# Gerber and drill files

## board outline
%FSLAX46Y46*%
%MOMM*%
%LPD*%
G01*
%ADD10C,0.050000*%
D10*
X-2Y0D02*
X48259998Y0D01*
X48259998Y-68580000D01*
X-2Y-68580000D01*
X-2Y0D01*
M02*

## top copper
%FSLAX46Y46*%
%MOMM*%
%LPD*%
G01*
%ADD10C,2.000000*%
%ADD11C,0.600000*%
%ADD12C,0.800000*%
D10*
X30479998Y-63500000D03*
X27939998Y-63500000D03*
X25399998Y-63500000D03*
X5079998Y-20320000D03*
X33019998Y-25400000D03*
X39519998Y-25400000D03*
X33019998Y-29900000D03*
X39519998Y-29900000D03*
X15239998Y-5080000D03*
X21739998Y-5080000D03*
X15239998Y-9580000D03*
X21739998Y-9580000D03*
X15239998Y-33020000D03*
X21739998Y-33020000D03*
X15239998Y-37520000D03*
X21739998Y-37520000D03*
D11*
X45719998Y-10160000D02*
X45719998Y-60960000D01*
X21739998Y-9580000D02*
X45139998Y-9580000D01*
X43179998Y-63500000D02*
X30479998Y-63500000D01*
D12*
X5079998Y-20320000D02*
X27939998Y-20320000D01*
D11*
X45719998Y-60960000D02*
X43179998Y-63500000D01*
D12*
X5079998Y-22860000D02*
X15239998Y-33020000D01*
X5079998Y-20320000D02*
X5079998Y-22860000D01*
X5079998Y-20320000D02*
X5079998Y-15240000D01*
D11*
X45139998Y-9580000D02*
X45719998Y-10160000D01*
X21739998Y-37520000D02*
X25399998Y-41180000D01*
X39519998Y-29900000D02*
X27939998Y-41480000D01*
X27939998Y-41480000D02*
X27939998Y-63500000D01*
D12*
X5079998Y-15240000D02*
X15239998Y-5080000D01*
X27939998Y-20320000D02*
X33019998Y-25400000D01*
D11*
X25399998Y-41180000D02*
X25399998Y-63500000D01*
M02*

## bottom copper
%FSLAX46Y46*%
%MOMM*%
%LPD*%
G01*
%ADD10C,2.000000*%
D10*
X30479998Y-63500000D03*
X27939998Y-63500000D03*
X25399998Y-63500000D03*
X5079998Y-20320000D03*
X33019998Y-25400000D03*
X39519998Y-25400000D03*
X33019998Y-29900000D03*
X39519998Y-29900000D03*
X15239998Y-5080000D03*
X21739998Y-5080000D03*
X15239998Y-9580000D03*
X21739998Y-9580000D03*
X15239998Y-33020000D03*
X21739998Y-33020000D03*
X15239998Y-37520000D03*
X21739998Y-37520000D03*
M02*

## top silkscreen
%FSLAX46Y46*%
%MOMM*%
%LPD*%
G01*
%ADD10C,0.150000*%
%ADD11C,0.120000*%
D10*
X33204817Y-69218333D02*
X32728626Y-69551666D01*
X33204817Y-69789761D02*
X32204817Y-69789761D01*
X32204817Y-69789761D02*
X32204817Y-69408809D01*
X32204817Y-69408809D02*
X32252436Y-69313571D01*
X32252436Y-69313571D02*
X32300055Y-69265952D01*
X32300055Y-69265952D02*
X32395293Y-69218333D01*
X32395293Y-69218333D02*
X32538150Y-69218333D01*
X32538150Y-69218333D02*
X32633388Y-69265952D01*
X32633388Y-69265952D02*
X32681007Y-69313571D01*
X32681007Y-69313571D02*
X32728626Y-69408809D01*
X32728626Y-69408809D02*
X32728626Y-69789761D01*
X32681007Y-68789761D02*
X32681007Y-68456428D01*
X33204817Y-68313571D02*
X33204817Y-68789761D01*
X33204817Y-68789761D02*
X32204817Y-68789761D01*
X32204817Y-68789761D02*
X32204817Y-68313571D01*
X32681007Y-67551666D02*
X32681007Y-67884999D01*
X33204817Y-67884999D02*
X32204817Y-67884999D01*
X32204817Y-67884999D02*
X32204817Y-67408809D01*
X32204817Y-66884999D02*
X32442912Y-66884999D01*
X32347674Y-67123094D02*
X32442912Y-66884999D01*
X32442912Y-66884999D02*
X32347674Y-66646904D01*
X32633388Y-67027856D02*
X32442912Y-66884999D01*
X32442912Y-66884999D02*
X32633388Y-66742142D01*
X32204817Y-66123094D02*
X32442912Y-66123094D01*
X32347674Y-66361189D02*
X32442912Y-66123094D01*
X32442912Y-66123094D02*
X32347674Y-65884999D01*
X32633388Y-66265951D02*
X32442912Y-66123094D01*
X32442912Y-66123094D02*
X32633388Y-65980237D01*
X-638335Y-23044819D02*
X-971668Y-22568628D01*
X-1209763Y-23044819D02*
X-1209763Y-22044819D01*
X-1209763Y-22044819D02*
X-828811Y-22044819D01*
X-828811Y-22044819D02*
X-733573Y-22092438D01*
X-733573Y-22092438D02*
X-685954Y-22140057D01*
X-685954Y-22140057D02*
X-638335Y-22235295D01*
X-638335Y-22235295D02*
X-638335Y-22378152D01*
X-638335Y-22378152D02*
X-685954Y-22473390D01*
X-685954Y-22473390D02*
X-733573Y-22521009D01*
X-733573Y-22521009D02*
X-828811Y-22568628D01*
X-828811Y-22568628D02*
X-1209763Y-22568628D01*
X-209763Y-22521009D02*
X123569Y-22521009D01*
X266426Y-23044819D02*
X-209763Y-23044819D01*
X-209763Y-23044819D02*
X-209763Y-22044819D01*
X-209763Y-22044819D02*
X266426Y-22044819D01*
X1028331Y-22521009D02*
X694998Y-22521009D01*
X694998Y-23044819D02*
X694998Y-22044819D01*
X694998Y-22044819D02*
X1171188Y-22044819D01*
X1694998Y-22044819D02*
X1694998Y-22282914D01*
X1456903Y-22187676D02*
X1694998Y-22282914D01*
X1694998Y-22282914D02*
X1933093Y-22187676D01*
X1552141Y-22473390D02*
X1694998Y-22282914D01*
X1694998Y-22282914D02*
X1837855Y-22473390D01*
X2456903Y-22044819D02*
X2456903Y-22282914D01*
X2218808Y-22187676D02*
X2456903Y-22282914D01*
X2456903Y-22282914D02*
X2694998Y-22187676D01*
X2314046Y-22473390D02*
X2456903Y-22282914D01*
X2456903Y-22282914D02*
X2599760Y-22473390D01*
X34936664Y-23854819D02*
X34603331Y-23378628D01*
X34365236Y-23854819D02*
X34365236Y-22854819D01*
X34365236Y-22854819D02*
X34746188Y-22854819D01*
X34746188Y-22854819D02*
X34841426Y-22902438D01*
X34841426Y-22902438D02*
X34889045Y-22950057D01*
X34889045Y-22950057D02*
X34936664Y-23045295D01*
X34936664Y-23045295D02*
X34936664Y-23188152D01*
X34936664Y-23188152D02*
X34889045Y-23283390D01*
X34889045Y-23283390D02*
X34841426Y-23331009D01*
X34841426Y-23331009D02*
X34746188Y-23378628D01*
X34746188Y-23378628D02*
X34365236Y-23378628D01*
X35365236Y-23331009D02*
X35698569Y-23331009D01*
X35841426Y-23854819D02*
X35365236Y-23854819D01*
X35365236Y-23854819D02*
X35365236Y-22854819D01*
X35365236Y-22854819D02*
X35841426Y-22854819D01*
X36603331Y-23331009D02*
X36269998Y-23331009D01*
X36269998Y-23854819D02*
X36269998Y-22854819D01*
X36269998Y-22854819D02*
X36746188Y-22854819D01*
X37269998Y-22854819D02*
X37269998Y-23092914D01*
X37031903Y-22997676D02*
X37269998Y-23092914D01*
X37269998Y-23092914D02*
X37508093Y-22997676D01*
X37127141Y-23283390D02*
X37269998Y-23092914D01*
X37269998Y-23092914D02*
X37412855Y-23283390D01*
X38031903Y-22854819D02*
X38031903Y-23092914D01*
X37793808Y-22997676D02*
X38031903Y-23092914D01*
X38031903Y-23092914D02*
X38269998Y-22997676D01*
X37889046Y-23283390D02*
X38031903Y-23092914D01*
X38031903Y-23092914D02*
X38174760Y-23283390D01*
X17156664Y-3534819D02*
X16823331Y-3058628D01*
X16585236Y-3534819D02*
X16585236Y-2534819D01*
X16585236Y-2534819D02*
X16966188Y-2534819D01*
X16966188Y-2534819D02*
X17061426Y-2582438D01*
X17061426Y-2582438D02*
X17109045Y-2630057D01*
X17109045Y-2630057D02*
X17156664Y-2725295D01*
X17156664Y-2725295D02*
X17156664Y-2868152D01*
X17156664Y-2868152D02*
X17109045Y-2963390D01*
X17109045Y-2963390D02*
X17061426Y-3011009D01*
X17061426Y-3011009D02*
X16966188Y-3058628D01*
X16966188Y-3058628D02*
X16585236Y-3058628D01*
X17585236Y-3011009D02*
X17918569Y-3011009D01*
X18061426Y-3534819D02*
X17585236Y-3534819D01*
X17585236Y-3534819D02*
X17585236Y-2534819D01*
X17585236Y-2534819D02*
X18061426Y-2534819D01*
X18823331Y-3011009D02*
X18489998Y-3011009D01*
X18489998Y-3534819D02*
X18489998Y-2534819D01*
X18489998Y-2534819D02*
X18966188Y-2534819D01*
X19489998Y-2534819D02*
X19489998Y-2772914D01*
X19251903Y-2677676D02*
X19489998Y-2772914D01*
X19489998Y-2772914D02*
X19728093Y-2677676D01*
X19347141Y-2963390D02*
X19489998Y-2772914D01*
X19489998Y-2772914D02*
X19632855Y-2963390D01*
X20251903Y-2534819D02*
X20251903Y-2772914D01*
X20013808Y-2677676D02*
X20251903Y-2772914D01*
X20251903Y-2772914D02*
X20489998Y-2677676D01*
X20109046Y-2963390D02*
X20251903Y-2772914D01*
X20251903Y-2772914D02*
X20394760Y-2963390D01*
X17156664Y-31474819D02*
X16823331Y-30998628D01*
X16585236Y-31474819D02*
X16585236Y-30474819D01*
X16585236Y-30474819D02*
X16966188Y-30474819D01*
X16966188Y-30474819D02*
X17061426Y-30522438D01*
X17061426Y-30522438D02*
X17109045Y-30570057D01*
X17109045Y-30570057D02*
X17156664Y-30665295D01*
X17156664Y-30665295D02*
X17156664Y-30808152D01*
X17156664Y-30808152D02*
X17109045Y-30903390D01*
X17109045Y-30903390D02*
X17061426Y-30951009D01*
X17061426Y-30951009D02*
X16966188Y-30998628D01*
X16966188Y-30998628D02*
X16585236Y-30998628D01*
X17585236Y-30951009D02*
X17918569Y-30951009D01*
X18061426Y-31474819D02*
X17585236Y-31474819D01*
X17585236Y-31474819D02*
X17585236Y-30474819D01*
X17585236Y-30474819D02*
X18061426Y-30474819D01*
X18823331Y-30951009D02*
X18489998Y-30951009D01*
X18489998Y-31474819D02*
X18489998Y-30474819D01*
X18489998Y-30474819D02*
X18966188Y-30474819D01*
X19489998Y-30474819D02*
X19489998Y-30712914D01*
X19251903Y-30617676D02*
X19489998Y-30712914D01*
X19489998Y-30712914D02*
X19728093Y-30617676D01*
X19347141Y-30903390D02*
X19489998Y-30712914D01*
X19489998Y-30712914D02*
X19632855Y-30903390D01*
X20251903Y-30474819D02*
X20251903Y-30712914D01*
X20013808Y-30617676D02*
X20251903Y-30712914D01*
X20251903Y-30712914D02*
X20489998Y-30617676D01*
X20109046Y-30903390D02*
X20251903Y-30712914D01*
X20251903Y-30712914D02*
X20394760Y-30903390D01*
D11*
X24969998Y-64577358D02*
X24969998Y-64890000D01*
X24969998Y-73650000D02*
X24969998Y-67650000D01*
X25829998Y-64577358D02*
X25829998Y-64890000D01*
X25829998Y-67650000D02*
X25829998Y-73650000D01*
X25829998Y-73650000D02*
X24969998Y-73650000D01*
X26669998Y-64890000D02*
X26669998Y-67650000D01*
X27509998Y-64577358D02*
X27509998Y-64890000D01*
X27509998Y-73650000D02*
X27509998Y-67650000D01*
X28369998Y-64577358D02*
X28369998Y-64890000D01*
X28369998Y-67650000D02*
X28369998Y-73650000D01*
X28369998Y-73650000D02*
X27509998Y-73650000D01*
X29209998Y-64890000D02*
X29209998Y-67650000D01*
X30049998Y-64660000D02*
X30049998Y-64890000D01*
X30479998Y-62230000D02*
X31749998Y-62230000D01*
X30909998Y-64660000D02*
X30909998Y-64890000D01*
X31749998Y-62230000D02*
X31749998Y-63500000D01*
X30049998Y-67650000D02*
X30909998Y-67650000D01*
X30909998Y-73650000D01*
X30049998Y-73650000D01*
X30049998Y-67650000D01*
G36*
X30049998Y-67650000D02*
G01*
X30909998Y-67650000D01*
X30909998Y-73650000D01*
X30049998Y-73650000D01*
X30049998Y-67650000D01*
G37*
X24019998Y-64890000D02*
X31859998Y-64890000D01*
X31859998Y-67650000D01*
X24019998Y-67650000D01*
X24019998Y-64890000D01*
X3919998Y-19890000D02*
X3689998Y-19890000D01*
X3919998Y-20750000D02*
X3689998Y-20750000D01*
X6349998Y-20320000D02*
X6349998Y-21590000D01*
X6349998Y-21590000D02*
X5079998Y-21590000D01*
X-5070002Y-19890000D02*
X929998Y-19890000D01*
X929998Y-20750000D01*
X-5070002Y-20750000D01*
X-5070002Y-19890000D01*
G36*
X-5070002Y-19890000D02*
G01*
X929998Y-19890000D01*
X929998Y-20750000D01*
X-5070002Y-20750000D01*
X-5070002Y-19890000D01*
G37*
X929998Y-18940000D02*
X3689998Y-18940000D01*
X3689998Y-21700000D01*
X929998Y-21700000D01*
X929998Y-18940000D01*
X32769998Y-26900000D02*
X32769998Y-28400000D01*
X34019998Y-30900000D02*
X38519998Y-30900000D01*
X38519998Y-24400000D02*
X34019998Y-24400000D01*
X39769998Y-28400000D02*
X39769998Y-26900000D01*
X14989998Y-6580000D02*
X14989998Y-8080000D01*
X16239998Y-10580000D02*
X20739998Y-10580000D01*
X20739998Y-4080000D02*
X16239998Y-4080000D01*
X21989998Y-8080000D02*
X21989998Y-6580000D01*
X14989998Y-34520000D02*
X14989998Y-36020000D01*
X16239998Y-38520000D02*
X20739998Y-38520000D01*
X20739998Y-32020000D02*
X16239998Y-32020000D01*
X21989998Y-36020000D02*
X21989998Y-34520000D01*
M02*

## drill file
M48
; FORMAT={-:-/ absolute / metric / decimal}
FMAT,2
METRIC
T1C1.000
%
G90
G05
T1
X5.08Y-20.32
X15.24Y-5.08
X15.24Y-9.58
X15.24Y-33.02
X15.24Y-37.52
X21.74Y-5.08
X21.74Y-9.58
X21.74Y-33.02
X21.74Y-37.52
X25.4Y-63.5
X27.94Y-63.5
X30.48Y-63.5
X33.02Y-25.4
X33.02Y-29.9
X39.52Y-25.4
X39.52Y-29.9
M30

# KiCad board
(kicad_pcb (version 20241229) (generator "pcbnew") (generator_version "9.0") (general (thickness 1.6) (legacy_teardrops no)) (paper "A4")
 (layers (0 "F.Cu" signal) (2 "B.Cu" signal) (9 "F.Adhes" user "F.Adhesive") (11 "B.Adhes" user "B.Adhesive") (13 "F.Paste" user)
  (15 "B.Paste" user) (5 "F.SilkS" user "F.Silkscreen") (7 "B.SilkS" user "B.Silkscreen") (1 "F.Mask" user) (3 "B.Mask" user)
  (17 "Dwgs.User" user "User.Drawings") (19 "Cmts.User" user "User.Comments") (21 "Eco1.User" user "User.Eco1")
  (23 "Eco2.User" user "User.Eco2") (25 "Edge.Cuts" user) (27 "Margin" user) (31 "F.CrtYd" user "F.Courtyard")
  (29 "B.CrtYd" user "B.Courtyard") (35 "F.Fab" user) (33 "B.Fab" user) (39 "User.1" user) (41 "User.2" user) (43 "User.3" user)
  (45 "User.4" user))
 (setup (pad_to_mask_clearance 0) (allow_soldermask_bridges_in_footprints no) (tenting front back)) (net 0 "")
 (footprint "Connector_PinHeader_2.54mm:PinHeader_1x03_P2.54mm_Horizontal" (layer "F.Cu") (at 30.479998 63.5 -90)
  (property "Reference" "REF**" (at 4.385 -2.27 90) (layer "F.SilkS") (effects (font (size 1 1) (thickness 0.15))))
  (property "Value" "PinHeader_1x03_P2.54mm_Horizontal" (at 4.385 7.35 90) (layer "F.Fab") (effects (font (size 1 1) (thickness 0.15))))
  (fp_line (start 1.077358 5.51) (end 1.39 5.51) (stroke (width 0.12) (type solid)) (layer "F.SilkS"))
  (fp_line (start 10.15 5.51) (end 4.15 5.51) (stroke (width 0.12) (type solid)) (layer "F.SilkS"))
  (fp_line (start 1.077358 4.65) (end 1.39 4.65) (stroke (width 0.12) (type solid)) (layer "F.SilkS"))
  (fp_line (start 4.15 4.65) (end 10.15 4.65) (stroke (width 0.12) (type solid)) (layer "F.SilkS"))
  (fp_line (start 10.15 4.65) (end 10.15 5.51) (stroke (width 0.12) (type solid)) (layer "F.SilkS"))
  (fp_line (start 1.39 3.81) (end 4.15 3.81) (stroke (width 0.12) (type solid)) (layer "F.SilkS"))
  (fp_line (start 1.077358 2.97) (end 1.39 2.97) (stroke (width 0.12) (type solid)) (layer "F.SilkS"))
  (fp_line (start 10.15 2.97) (end 4.15 2.97) (stroke (width 0.12) (type solid)) (layer "F.SilkS"))
  (fp_line (start 1.077358 2.11) (end 1.39 2.11) (stroke (width 0.12) (type solid)) (layer "F.SilkS"))
  (fp_line (start 4.15 2.11) (end 10.15 2.11) (stroke (width 0.12) (type solid)) (layer "F.SilkS"))
  (fp_line (start 10.15 2.11) (end 10.15 2.97) (stroke (width 0.12) (type solid)) (layer "F.SilkS"))
  (fp_line (start 1.39 1.27) (end 4.15 1.27) (stroke (width 0.12) (type solid)) (layer "F.SilkS"))
  (fp_line (start 1.16 0.43) (end 1.39 0.43) (stroke (width 0.12) (type solid)) (layer "F.SilkS"))
  (fp_line (start -1.27 0) (end -1.27 -1.27) (stroke (width 0.12) (type solid)) (layer "F.SilkS"))
  (fp_line (start 1.16 -0.43) (end 1.39 -0.43) (stroke (width 0.12) (type solid)) (layer "F.SilkS"))
  (fp_line (start -1.27 -1.27) (end 0 -1.27) (stroke (width 0.12) (type solid)) (layer "F.SilkS"))
  (fp_rect (start 4.15 -0.43) (end 10.15 0.43) (stroke (width 0.12) (type solid)) (fill yes) (layer "F.SilkS"))
  (fp_rect (start 1.39 -1.38) (end 4.15 6.46) (stroke (width 0.12) (type solid)) (fill no) (layer "F.SilkS"))
  (pad "1" thru_hole circle (at 0 0 270) (size 2 2) (drill 1) (layers "*.Cu" "*.Mask") (remove_unused_layers no))
  (pad "2" thru_hole circle (at 0 2.54 270) (size 2 2) (drill 1) (layers "*.Cu" "*.Mask") (remove_unused_layers no))
  (pad "3" thru_hole circle (at 0 5.08 270) (size 2 2) (drill 1) (layers "*.Cu" "*.Mask") (remove_unused_layers no)))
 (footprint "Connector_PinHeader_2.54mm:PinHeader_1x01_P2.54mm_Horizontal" (layer "F.Cu") (at 5.079998 20.32 180)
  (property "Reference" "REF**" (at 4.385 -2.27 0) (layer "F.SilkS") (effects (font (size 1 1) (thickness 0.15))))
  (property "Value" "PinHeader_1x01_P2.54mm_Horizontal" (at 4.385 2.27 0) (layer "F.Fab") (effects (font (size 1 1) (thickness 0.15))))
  (fp_line (start 1.16 0.43) (end 1.39 0.43) (stroke (width 0.12) (type solid)) (layer "F.SilkS"))
  (fp_line (start 1.16 -0.43) (end 1.39 -0.43) (stroke (width 0.12) (type solid)) (layer "F.SilkS"))
  (fp_line (start -1.27 0) (end -1.27 -1.27) (stroke (width 0.12) (type solid)) (layer "F.SilkS"))
  (fp_line (start -1.27 -1.27) (end 0 -1.27) (stroke (width 0.12) (type solid)) (layer "F.SilkS"))
  (fp_rect (start 4.15 -0.43) (end 10.15 0.43) (stroke (width 0.12) (type solid)) (fill yes) (layer "F.SilkS"))
  (fp_rect (start 1.39 -1.38) (end 4.15 1.38) (stroke (width 0.12) (type solid)) (fill no) (layer "F.SilkS"))
  (pad "1" thru_hole circle (at 0 0 180) (size 2 2) (drill 1) (layers "*.Cu" "*.Mask") (remove_unused_layers no)))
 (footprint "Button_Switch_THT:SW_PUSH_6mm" (layer "F.Cu") (at 33.019998 25.4)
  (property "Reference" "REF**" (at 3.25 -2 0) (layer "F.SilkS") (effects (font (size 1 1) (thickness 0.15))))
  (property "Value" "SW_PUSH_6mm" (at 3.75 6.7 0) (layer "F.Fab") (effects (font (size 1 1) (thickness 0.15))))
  (fp_line (start -0.25 1.5) (end -0.25 3) (stroke (width 0.12) (type solid)) (layer "F.SilkS"))
  (fp_line (start 1 5.5) (end 5.5 5.5) (stroke (width 0.12) (type solid)) (layer "F.SilkS"))
  (fp_line (start 5.5 -1) (end 1 -1) (stroke (width 0.12) (type solid)) (layer "F.SilkS"))
  (fp_line (start 6.75 3) (end 6.75 1.5) (stroke (width 0.12) (type solid)) (layer "F.SilkS"))
  (pad "1" thru_hole circle (at 0 0 90) (size 2 2) (drill 1) (layers "*.Cu" "*.Mask") (remove_unused_layers no))
  (pad "1" thru_hole circle (at 6.5 0 90) (size 2 2) (drill 1) (layers "*.Cu" "*.Mask") (remove_unused_layers no))
  (pad "2" thru_hole circle (at 0 4.5 90) (size 2 2) (drill 1) (layers "*.Cu" "*.Mask") (remove_unused_layers no))
  (pad "2" thru_hole circle (at 6.5 4.5 90) (size 2 2) (drill 1) (layers "*.Cu" "*.Mask") (remove_unused_layers no)))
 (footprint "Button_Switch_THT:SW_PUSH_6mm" (layer "F.Cu") (at 15.239998 5.08)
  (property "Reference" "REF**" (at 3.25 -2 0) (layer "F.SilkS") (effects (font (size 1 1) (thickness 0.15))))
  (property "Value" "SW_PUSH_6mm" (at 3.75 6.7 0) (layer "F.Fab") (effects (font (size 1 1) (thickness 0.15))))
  (fp_line (start -0.25 1.5) (end -0.25 3) (stroke (width 0.12) (type solid)) (layer "F.SilkS"))
  (fp_line (start 1 5.5) (end 5.5 5.5) (stroke (width 0.12) (type solid)) (layer "F.SilkS"))
  (fp_line (start 5.5 -1) (end 1 -1) (stroke (width 0.12) (type solid)) (layer "F.SilkS"))
  (fp_line (start 6.75 3) (end 6.75 1.5) (stroke (width 0.12) (type solid)) (layer "F.SilkS"))
  (pad "1" thru_hole circle (at 0 0 90) (size 2 2) (drill 1) (layers "*.Cu" "*.Mask") (remove_unused_layers no))
  (pad "1" thru_hole circle (at 6.5 0 90) (size 2 2) (drill 1) (layers "*.Cu" "*.Mask") (remove_unused_layers no))
  (pad "2" thru_hole circle (at 0 4.5 90) (size 2 2) (drill 1) (layers "*.Cu" "*.Mask") (remove_unused_layers no))
  (pad "2" thru_hole circle (at 6.5 4.5 90) (size 2 2) (drill 1) (layers "*.Cu" "*.Mask") (remove_unused_layers no)))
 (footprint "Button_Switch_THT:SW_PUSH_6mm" (layer "F.Cu") (at 15.239998 33.02)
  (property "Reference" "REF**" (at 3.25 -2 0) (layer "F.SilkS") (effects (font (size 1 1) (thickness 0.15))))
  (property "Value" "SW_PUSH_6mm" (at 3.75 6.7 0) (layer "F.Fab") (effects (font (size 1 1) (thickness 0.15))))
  (fp_line (start -0.25 1.5) (end -0.25 3) (stroke (width 0.12) (type solid)) (layer "F.SilkS"))
  (fp_line (start 1 5.5) (end 5.5 5.5) (stroke (width 0.12) (type solid)) (layer "F.SilkS"))
  (fp_line (start 5.5 -1) (end 1 -1) (stroke (width 0.12) (type solid)) (layer "F.SilkS"))
  (fp_line (start 6.75 3) (end 6.75 1.5) (stroke (width 0.12) (type solid)) (layer "F.SilkS"))
  (pad "1" thru_hole circle (at 0 0 90) (size 2 2) (drill 1) (layers "*.Cu" "*.Mask") (remove_unused_layers no))
  (pad "1" thru_hole circle (at 6.5 0 90) (size 2 2) (drill 1) (layers "*.Cu" "*.Mask") (remove_unused_layers no))
  (pad "2" thru_hole circle (at 0 4.5 90) (size 2 2) (drill 1) (layers "*.Cu" "*.Mask") (remove_unused_layers no))
  (pad "2" thru_hole circle (at 6.5 4.5 90) (size 2 2) (drill 1) (layers "*.Cu" "*.Mask") (remove_unused_layers no)))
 (gr_rect (start -0.000002 0) (end 48.259998 68.58) (stroke (width 0.05) (type default)) (fill no) (layer "Edge.Cuts"))
 (segment (start 45.719998 10.16) (end 45.719998 60.96) (width 0.6) (layer "F.Cu") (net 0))
 (segment (start 21.739998 9.58) (end 45.139998 9.58) (width 0.6) (layer "F.Cu") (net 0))
 (segment (start 43.179998 63.5) (end 30.479998 63.5) (width 0.6) (layer "F.Cu") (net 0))
 (segment (start 5.079998 20.32) (end 27.939998 20.32) (width 0.8) (layer "F.Cu") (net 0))
 (segment (start 45.719998 60.96) (end 43.179998 63.5) (width 0.6) (layer "F.Cu") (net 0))
 (segment (start 5.079998 22.86) (end 15.239998 33.02) (width 0.8) (layer "F.Cu") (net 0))
 (segment (start 5.079998 20.32) (end 5.079998 22.86) (width 0.8) (layer "F.Cu") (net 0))
 (segment (start 5.079998 20.32) (end 5.079998 15.24) (width 0.8) (layer "F.Cu") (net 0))
 (segment (start 45.139998 9.58) (end 45.719998 10.16) (width 0.6) (layer "F.Cu") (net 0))
 (segment (start 21.739998 37.52) (end 25.399998 41.18) (width 0.6) (layer "F.Cu") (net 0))
 (segment (start 39.519998 29.9) (end 27.939998 41.48) (width 0.6) (layer "F.Cu") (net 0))
 (segment (start 27.939998 41.48) (end 27.939998 63.5) (width 0.6) (layer "F.Cu") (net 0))
 (segment (start 5.079998 15.24) (end 15.239998 5.08) (width 0.8) (layer "F.Cu") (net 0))
 (segment (start 27.939998 20.32) (end 33.019998 25.4) (width 0.8) (layer "F.Cu") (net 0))
 (segment (start 25.399998 41.18) (end 25.399998 63.5) (width 0.6) (layer "F.Cu") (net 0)))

